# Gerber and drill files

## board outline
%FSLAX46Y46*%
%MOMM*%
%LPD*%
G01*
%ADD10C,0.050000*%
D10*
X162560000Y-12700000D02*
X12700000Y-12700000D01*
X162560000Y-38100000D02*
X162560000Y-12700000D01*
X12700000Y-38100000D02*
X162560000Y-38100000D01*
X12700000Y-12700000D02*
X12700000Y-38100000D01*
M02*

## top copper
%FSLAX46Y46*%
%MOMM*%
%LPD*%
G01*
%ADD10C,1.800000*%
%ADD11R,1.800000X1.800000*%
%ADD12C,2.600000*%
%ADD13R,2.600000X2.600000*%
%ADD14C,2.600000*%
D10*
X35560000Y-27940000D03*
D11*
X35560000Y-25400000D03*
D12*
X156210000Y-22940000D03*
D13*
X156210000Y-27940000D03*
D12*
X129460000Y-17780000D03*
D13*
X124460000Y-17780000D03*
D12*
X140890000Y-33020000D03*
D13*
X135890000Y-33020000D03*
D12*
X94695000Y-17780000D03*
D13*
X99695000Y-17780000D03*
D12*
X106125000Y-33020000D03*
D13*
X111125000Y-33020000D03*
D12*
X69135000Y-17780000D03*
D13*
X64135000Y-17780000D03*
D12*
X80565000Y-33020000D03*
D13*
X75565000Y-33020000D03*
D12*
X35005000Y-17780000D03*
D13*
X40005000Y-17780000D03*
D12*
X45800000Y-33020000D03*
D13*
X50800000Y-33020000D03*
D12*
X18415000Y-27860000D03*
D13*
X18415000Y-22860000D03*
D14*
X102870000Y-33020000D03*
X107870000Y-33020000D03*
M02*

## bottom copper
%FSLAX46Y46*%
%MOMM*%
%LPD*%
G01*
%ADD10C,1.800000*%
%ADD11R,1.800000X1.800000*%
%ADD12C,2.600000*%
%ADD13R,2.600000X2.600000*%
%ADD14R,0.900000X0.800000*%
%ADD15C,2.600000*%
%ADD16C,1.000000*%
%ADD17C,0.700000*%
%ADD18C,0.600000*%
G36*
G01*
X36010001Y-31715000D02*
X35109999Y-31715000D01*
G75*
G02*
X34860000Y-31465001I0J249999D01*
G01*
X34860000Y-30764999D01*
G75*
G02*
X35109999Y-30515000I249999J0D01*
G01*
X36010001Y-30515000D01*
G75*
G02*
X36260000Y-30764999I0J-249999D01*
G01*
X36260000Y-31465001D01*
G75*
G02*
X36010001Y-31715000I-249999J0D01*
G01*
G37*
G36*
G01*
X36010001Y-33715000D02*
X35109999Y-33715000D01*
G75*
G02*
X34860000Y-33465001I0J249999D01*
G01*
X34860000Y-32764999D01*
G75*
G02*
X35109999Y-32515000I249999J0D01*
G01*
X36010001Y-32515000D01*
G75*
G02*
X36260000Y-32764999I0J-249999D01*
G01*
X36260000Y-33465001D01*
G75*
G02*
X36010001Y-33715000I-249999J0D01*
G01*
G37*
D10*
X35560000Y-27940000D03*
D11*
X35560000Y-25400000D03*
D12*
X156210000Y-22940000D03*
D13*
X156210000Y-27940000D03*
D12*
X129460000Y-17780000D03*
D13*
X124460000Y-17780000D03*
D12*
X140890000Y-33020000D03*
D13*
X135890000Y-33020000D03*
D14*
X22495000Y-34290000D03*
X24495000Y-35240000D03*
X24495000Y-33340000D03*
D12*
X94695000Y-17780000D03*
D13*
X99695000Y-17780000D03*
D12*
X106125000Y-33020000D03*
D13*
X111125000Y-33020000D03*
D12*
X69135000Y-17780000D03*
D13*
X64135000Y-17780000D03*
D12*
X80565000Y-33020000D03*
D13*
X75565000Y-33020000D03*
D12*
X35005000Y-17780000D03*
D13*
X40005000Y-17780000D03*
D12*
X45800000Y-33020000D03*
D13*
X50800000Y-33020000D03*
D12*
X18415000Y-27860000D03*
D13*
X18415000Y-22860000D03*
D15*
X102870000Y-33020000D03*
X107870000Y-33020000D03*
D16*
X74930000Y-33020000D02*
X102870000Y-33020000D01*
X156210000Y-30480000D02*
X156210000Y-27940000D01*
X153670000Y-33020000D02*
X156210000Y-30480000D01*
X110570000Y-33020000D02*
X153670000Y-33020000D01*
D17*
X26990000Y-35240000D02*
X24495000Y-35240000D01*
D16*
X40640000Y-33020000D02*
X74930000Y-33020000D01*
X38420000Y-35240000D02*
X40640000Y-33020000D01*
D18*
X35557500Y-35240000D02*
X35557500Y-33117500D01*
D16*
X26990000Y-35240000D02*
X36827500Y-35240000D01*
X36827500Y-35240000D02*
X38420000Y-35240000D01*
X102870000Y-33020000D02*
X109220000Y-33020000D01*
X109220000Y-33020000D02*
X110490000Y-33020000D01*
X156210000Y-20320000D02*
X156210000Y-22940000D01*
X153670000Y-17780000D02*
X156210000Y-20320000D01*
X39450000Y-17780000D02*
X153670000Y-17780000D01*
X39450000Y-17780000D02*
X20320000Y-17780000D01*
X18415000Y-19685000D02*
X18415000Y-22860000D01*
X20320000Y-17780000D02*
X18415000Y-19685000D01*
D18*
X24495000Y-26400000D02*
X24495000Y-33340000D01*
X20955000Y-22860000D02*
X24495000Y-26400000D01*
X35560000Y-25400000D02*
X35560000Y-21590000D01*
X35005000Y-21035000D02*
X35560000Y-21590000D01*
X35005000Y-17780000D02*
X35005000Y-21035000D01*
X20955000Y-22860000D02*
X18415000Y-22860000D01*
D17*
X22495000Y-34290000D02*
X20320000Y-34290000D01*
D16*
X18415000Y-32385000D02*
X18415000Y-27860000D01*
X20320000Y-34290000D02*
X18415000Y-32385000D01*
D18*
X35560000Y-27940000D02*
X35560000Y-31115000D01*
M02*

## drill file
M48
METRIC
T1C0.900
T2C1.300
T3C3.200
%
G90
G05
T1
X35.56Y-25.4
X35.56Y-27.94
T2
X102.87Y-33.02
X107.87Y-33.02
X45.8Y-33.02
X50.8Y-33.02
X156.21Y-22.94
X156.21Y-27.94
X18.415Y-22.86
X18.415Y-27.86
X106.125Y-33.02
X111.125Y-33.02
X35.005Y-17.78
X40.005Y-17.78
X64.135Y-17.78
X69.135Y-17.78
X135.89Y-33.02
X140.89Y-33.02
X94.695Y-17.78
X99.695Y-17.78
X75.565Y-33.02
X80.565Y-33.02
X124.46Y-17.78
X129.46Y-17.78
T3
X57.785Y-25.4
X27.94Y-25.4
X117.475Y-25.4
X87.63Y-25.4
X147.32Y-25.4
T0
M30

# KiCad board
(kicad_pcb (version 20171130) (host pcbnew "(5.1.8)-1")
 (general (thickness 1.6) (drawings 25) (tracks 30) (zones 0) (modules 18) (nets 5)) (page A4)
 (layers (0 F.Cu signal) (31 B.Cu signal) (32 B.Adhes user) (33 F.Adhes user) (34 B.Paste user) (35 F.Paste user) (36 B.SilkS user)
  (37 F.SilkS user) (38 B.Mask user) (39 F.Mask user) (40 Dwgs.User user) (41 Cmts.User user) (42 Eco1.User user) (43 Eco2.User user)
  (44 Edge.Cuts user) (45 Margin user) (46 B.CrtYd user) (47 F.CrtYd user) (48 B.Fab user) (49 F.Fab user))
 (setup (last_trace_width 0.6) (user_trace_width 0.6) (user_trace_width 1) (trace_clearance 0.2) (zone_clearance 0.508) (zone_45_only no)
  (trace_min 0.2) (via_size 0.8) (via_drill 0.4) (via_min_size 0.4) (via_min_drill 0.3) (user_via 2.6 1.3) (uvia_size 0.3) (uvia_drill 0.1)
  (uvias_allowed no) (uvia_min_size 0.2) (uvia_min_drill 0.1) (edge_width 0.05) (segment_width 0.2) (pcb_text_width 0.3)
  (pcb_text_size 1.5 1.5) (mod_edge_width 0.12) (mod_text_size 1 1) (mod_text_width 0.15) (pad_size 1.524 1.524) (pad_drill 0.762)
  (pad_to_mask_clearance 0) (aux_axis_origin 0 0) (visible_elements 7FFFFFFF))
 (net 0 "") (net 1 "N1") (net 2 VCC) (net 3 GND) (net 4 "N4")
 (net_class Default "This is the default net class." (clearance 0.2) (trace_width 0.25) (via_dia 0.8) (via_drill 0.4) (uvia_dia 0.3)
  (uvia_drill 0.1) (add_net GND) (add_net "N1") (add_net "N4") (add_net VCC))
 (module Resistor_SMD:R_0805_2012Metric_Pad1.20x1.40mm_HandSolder (layer B.Cu) (at 35.56 32.115 90)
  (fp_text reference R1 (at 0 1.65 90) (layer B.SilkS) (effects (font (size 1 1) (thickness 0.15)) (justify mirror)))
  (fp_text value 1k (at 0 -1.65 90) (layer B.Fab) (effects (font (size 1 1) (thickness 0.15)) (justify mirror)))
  (pad 2 smd roundrect (at 1 0 90) (size 1.2 1.4) (layers B.Cu B.Paste B.Mask) (roundrect_rratio 0.2083325) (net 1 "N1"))
  (pad 1 smd roundrect (at -1 0 90) (size 1.2 1.4) (layers B.Cu B.Paste B.Mask) (roundrect_rratio 0.2083325) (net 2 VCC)))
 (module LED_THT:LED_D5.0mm (layer F.Cu) (at 35.56 25.4 270)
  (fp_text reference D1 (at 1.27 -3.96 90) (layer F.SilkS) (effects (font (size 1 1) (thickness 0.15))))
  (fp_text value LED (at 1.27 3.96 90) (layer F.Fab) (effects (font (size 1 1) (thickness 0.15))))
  (pad 2 thru_hole circle (at 2.54 0 270) (size 1.8 1.8) (drill 0.9) (layers *.Cu *.Mask) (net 1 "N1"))
  (pad 1 thru_hole rect (at 0 0 270) (size 1.8 1.8) (drill 0.9) (layers *.Cu *.Mask) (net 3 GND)))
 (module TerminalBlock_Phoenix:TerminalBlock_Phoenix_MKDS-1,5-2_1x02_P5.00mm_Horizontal (layer F.Cu) (at 156.21 27.94 90)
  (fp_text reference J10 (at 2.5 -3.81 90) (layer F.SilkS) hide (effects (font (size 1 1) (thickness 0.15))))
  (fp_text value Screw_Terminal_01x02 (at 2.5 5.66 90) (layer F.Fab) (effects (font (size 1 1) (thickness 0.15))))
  (pad 2 thru_hole circle (at 5 0 90) (size 2.6 2.6) (drill 1.3) (layers *.Cu *.Mask) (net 3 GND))
  (pad 1 thru_hole rect (at 0 0 90) (size 2.6 2.6) (drill 1.3) (layers *.Cu *.Mask) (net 2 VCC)))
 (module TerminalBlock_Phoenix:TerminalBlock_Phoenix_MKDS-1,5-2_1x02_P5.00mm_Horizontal (layer F.Cu) (at 124.46 17.78)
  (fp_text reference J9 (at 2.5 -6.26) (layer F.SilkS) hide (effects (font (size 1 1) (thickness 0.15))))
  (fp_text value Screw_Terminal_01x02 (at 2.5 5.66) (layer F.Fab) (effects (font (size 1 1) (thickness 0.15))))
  (pad 2 thru_hole circle (at 5 0) (size 2.6 2.6) (drill 1.3) (layers *.Cu *.Mask) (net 3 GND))
  (pad 1 thru_hole rect (at 0 0) (size 2.6 2.6) (drill 1.3) (layers *.Cu *.Mask) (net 3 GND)))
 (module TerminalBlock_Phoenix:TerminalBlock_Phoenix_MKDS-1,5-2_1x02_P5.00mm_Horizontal (layer F.Cu) (at 135.89 33.02)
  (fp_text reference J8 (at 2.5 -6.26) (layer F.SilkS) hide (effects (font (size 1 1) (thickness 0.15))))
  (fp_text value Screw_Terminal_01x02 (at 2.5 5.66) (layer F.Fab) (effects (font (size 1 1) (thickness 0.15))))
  (pad 2 thru_hole circle (at 5 0) (size 2.6 2.6) (drill 1.3) (layers *.Cu *.Mask) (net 2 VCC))
  (pad 1 thru_hole rect (at 0 0) (size 2.6 2.6) (drill 1.3) (layers *.Cu *.Mask) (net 2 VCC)))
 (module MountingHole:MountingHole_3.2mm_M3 (layer F.Cu) (at 147.32 25.4)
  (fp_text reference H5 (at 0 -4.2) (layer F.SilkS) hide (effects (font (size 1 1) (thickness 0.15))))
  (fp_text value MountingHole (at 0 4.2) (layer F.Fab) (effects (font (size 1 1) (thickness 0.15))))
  (pad 1 np_thru_hole circle (at 0 0) (size 3.2 3.2) (drill 3.2) (layers *.Cu *.Mask)))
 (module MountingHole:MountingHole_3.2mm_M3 (layer F.Cu) (at 117.475 25.4)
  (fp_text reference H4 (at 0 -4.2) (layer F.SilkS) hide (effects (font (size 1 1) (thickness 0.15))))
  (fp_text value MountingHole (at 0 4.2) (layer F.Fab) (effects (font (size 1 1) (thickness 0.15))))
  (pad 1 np_thru_hole circle (at 0 0) (size 3.2 3.2) (drill 3.2) (layers *.Cu *.Mask)))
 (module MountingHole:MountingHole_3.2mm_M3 (layer F.Cu) (at 87.63 25.4)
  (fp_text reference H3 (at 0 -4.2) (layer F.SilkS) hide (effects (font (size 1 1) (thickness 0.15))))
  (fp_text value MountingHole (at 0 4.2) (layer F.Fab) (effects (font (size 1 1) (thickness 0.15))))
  (pad 1 np_thru_hole circle (at 0 0) (size 3.2 3.2) (drill 3.2) (layers *.Cu *.Mask)))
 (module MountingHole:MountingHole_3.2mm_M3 (layer F.Cu) (at 57.785 25.4)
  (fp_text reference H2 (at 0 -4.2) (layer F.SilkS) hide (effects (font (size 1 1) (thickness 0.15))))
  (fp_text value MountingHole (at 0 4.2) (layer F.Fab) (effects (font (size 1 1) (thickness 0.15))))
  (pad 1 np_thru_hole circle (at 0 0) (size 3.2 3.2) (drill 3.2) (layers *.Cu *.Mask)))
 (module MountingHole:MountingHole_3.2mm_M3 (layer F.Cu) (at 27.94 25.4)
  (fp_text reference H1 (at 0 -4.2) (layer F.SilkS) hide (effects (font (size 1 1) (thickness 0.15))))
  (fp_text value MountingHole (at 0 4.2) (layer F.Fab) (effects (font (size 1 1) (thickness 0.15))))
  (pad 1 np_thru_hole circle (at 0 0) (size 3.2 3.2) (drill 3.2) (layers *.Cu *.Mask)))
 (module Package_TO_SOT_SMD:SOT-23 (layer B.Cu) (at 23.495 34.29 180)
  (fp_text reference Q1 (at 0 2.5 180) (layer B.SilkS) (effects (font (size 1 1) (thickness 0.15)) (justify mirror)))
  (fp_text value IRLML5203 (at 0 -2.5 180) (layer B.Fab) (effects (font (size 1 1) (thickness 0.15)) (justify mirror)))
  (pad 3 smd rect (at 1 0 180) (size 0.9 0.8) (layers B.Cu B.Paste B.Mask) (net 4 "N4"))
  (pad 2 smd rect (at -1 -0.95 180) (size 0.9 0.8) (layers B.Cu B.Paste B.Mask) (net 2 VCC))
  (pad 1 smd rect (at -1 0.95 180) (size 0.9 0.8) (layers B.Cu B.Paste B.Mask) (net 3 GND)))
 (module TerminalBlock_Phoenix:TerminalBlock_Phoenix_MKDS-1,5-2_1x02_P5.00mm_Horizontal (layer F.Cu) (at 99.695 17.78 180)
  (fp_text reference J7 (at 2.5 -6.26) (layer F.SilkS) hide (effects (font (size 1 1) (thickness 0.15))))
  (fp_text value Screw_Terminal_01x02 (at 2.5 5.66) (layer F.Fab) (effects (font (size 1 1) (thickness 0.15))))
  (pad 2 thru_hole circle (at 5 0 180) (size 2.6 2.6) (drill 1.3) (layers *.Cu *.Mask) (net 3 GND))
  (pad 1 thru_hole rect (at 0 0 180) (size 2.6 2.6) (drill 1.3) (layers *.Cu *.Mask) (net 3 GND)))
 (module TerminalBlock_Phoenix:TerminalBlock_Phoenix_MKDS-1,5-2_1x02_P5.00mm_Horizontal (layer F.Cu) (at 111.125 33.02 180)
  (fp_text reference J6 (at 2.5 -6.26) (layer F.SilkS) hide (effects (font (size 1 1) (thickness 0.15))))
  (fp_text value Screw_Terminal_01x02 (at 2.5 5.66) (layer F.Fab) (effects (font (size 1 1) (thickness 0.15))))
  (pad 2 thru_hole circle (at 5 0 180) (size 2.6 2.6) (drill 1.3) (layers *.Cu *.Mask) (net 2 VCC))
  (pad 1 thru_hole rect (at 0 0 180) (size 2.6 2.6) (drill 1.3) (layers *.Cu *.Mask) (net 2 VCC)))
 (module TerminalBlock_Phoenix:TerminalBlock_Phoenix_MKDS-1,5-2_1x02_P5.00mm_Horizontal (layer F.Cu) (at 64.135 17.78)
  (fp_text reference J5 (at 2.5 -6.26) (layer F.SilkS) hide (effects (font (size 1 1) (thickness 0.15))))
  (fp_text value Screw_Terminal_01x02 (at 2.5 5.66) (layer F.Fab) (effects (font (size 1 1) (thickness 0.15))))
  (pad 2 thru_hole circle (at 5 0) (size 2.6 2.6) (drill 1.3) (layers *.Cu *.Mask) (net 3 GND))
  (pad 1 thru_hole rect (at 0 0) (size 2.6 2.6) (drill 1.3) (layers *.Cu *.Mask) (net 3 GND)))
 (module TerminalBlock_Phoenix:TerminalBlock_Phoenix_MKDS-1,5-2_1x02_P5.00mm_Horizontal (layer F.Cu) (at 75.565 33.02)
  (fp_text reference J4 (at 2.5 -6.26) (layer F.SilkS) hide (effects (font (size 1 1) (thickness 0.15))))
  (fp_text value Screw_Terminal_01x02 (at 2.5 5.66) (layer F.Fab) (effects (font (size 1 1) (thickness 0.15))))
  (pad 2 thru_hole circle (at 5 0) (size 2.6 2.6) (drill 1.3) (layers *.Cu *.Mask) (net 2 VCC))
  (pad 1 thru_hole rect (at 0 0) (size 2.6 2.6) (drill 1.3) (layers *.Cu *.Mask) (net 2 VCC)))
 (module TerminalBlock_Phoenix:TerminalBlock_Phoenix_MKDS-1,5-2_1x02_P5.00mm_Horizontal (layer F.Cu) (at 40.005 17.78 180)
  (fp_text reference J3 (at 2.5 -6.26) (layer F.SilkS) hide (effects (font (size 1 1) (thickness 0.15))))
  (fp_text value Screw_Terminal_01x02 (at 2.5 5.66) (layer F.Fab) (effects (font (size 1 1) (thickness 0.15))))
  (pad 2 thru_hole circle (at 5 0 180) (size 2.6 2.6) (drill 1.3) (layers *.Cu *.Mask) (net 3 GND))
  (pad 1 thru_hole rect (at 0 0 180) (size 2.6 2.6) (drill 1.3) (layers *.Cu *.Mask) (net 3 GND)))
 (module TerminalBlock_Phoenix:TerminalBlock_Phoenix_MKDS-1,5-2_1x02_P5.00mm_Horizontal (layer F.Cu) (at 50.8 33.02 180)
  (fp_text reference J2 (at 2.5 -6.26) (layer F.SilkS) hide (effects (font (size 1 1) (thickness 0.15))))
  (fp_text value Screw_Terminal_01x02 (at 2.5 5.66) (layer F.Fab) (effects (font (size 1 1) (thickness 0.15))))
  (pad 2 thru_hole circle (at 5 0 180) (size 2.6 2.6) (drill 1.3) (layers *.Cu *.Mask) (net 2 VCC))
  (pad 1 thru_hole rect (at 0 0 180) (size 2.6 2.6) (drill 1.3) (layers *.Cu *.Mask) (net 2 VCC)))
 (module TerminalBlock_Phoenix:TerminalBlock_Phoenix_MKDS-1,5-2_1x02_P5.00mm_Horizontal (layer F.Cu) (at 18.415 22.86 270)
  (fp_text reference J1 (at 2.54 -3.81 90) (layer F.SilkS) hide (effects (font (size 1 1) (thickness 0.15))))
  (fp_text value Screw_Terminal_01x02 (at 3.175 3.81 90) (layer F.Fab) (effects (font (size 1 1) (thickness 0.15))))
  (pad 2 thru_hole circle (at 5 0 270) (size 2.6 2.6) (drill 1.3) (layers *.Cu *.Mask) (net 4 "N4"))
  (pad 1 thru_hole rect (at 0 0 270) (size 2.6 2.6) (drill 1.3) (layers *.Cu *.Mask) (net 3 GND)))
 (gr_line (start 162.56 12.7) (end 12.7 12.7) (layer Edge.Cuts) (width 0.05))
 (gr_line (start 162.56 38.1) (end 162.56 12.7) (layer Edge.Cuts) (width 0.05))
 (gr_line (start 12.7 38.1) (end 162.56 38.1) (layer Edge.Cuts) (width 0.05))
 (gr_line (start 12.7 12.7) (end 12.7 38.1) (layer Edge.Cuts) (width 0.05))
 (segment (start 74.93 33.02) (end 102.87 33.02) (width 1) (layer B.Cu) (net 2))
 (segment (start 156.21 30.48) (end 156.21 27.94) (width 1) (layer B.Cu) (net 2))
 (segment (start 153.67 33.02) (end 156.21 30.48) (width 1) (layer B.Cu) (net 2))
 (segment (start 110.57 33.02) (end 153.67 33.02) (width 1) (layer B.Cu) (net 2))
 (segment (start 26.99 35.24) (end 24.495 35.24) (width 0.7) (layer B.Cu) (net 2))
 (segment (start 40.64 33.02) (end 74.93 33.02) (width 1) (layer B.Cu) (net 2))
 (segment (start 38.42 35.24) (end 40.64 33.02) (width 1) (layer B.Cu) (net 2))
 (segment (start 35.5575 35.24) (end 35.5575 33.1175) (width 0.6) (layer B.Cu) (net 2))
 (segment (start 26.99 35.24) (end 36.8275 35.24) (width 1) (layer B.Cu) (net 2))
 (segment (start 36.8275 35.24) (end 38.42 35.24) (width 1) (layer B.Cu) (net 2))
 (segment (start 102.87 33.02) (end 109.22 33.02) (width 1) (layer B.Cu) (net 2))
 (via (at 102.87 33.02) (size 2.6) (drill 1.3) (layers F.Cu B.Cu) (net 2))
 (segment (start 109.22 33.02) (end 110.49 33.02) (width 1) (layer B.Cu) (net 2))
 (via (at 107.87 33.02) (size 2.6) (drill 1.3) (layers F.Cu B.Cu) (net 2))
 (segment (start 156.21 20.32) (end 156.21 22.94) (width 1) (layer B.Cu) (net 3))
 (segment (start 153.67 17.78) (end 156.21 20.32) (width 1) (layer B.Cu) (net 3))
 (segment (start 39.45 17.78) (end 153.67 17.78) (width 1) (layer B.Cu) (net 3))
 (segment (start 39.45 17.78) (end 20.32 17.78) (width 1) (layer B.Cu) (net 3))
 (segment (start 18.415 19.685) (end 18.415 22.86) (width 1) (layer B.Cu) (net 3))
 (segment (start 20.32 17.78) (end 18.415 19.685) (width 1) (layer B.Cu) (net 3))
 (segment (start 24.495 26.4) (end 24.495 33.34) (width 0.6) (layer B.Cu) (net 3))
 (segment (start 20.955 22.86) (end 24.495 26.4) (width 0.6) (layer B.Cu) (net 3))
 (segment (start 35.56 25.4) (end 35.56 21.59) (width 0.6) (layer B.Cu) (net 3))
 (segment (start 35.005 21.035) (end 35.56 21.59) (width 0.6) (layer B.Cu) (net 3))
 (segment (start 35.005 17.78) (end 35.005 21.035) (width 0.6) (layer B.Cu) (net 3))
 (segment (start 20.955 22.86) (end 18.415 22.86) (width 0.6) (layer B.Cu) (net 3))
 (segment (start 22.495 34.29) (end 20.32 34.29) (width 0.7) (layer B.Cu) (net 4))
 (segment (start 18.415 32.385) (end 18.415 27.86) (width 1) (layer B.Cu) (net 4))
 (segment (start 20.32 34.29) (end 18.415 32.385) (width 1) (layer B.Cu) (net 4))
 (segment (start 35.56 27.94) (end 35.56 31.115) (width 0.6) (layer B.Cu) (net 1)))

